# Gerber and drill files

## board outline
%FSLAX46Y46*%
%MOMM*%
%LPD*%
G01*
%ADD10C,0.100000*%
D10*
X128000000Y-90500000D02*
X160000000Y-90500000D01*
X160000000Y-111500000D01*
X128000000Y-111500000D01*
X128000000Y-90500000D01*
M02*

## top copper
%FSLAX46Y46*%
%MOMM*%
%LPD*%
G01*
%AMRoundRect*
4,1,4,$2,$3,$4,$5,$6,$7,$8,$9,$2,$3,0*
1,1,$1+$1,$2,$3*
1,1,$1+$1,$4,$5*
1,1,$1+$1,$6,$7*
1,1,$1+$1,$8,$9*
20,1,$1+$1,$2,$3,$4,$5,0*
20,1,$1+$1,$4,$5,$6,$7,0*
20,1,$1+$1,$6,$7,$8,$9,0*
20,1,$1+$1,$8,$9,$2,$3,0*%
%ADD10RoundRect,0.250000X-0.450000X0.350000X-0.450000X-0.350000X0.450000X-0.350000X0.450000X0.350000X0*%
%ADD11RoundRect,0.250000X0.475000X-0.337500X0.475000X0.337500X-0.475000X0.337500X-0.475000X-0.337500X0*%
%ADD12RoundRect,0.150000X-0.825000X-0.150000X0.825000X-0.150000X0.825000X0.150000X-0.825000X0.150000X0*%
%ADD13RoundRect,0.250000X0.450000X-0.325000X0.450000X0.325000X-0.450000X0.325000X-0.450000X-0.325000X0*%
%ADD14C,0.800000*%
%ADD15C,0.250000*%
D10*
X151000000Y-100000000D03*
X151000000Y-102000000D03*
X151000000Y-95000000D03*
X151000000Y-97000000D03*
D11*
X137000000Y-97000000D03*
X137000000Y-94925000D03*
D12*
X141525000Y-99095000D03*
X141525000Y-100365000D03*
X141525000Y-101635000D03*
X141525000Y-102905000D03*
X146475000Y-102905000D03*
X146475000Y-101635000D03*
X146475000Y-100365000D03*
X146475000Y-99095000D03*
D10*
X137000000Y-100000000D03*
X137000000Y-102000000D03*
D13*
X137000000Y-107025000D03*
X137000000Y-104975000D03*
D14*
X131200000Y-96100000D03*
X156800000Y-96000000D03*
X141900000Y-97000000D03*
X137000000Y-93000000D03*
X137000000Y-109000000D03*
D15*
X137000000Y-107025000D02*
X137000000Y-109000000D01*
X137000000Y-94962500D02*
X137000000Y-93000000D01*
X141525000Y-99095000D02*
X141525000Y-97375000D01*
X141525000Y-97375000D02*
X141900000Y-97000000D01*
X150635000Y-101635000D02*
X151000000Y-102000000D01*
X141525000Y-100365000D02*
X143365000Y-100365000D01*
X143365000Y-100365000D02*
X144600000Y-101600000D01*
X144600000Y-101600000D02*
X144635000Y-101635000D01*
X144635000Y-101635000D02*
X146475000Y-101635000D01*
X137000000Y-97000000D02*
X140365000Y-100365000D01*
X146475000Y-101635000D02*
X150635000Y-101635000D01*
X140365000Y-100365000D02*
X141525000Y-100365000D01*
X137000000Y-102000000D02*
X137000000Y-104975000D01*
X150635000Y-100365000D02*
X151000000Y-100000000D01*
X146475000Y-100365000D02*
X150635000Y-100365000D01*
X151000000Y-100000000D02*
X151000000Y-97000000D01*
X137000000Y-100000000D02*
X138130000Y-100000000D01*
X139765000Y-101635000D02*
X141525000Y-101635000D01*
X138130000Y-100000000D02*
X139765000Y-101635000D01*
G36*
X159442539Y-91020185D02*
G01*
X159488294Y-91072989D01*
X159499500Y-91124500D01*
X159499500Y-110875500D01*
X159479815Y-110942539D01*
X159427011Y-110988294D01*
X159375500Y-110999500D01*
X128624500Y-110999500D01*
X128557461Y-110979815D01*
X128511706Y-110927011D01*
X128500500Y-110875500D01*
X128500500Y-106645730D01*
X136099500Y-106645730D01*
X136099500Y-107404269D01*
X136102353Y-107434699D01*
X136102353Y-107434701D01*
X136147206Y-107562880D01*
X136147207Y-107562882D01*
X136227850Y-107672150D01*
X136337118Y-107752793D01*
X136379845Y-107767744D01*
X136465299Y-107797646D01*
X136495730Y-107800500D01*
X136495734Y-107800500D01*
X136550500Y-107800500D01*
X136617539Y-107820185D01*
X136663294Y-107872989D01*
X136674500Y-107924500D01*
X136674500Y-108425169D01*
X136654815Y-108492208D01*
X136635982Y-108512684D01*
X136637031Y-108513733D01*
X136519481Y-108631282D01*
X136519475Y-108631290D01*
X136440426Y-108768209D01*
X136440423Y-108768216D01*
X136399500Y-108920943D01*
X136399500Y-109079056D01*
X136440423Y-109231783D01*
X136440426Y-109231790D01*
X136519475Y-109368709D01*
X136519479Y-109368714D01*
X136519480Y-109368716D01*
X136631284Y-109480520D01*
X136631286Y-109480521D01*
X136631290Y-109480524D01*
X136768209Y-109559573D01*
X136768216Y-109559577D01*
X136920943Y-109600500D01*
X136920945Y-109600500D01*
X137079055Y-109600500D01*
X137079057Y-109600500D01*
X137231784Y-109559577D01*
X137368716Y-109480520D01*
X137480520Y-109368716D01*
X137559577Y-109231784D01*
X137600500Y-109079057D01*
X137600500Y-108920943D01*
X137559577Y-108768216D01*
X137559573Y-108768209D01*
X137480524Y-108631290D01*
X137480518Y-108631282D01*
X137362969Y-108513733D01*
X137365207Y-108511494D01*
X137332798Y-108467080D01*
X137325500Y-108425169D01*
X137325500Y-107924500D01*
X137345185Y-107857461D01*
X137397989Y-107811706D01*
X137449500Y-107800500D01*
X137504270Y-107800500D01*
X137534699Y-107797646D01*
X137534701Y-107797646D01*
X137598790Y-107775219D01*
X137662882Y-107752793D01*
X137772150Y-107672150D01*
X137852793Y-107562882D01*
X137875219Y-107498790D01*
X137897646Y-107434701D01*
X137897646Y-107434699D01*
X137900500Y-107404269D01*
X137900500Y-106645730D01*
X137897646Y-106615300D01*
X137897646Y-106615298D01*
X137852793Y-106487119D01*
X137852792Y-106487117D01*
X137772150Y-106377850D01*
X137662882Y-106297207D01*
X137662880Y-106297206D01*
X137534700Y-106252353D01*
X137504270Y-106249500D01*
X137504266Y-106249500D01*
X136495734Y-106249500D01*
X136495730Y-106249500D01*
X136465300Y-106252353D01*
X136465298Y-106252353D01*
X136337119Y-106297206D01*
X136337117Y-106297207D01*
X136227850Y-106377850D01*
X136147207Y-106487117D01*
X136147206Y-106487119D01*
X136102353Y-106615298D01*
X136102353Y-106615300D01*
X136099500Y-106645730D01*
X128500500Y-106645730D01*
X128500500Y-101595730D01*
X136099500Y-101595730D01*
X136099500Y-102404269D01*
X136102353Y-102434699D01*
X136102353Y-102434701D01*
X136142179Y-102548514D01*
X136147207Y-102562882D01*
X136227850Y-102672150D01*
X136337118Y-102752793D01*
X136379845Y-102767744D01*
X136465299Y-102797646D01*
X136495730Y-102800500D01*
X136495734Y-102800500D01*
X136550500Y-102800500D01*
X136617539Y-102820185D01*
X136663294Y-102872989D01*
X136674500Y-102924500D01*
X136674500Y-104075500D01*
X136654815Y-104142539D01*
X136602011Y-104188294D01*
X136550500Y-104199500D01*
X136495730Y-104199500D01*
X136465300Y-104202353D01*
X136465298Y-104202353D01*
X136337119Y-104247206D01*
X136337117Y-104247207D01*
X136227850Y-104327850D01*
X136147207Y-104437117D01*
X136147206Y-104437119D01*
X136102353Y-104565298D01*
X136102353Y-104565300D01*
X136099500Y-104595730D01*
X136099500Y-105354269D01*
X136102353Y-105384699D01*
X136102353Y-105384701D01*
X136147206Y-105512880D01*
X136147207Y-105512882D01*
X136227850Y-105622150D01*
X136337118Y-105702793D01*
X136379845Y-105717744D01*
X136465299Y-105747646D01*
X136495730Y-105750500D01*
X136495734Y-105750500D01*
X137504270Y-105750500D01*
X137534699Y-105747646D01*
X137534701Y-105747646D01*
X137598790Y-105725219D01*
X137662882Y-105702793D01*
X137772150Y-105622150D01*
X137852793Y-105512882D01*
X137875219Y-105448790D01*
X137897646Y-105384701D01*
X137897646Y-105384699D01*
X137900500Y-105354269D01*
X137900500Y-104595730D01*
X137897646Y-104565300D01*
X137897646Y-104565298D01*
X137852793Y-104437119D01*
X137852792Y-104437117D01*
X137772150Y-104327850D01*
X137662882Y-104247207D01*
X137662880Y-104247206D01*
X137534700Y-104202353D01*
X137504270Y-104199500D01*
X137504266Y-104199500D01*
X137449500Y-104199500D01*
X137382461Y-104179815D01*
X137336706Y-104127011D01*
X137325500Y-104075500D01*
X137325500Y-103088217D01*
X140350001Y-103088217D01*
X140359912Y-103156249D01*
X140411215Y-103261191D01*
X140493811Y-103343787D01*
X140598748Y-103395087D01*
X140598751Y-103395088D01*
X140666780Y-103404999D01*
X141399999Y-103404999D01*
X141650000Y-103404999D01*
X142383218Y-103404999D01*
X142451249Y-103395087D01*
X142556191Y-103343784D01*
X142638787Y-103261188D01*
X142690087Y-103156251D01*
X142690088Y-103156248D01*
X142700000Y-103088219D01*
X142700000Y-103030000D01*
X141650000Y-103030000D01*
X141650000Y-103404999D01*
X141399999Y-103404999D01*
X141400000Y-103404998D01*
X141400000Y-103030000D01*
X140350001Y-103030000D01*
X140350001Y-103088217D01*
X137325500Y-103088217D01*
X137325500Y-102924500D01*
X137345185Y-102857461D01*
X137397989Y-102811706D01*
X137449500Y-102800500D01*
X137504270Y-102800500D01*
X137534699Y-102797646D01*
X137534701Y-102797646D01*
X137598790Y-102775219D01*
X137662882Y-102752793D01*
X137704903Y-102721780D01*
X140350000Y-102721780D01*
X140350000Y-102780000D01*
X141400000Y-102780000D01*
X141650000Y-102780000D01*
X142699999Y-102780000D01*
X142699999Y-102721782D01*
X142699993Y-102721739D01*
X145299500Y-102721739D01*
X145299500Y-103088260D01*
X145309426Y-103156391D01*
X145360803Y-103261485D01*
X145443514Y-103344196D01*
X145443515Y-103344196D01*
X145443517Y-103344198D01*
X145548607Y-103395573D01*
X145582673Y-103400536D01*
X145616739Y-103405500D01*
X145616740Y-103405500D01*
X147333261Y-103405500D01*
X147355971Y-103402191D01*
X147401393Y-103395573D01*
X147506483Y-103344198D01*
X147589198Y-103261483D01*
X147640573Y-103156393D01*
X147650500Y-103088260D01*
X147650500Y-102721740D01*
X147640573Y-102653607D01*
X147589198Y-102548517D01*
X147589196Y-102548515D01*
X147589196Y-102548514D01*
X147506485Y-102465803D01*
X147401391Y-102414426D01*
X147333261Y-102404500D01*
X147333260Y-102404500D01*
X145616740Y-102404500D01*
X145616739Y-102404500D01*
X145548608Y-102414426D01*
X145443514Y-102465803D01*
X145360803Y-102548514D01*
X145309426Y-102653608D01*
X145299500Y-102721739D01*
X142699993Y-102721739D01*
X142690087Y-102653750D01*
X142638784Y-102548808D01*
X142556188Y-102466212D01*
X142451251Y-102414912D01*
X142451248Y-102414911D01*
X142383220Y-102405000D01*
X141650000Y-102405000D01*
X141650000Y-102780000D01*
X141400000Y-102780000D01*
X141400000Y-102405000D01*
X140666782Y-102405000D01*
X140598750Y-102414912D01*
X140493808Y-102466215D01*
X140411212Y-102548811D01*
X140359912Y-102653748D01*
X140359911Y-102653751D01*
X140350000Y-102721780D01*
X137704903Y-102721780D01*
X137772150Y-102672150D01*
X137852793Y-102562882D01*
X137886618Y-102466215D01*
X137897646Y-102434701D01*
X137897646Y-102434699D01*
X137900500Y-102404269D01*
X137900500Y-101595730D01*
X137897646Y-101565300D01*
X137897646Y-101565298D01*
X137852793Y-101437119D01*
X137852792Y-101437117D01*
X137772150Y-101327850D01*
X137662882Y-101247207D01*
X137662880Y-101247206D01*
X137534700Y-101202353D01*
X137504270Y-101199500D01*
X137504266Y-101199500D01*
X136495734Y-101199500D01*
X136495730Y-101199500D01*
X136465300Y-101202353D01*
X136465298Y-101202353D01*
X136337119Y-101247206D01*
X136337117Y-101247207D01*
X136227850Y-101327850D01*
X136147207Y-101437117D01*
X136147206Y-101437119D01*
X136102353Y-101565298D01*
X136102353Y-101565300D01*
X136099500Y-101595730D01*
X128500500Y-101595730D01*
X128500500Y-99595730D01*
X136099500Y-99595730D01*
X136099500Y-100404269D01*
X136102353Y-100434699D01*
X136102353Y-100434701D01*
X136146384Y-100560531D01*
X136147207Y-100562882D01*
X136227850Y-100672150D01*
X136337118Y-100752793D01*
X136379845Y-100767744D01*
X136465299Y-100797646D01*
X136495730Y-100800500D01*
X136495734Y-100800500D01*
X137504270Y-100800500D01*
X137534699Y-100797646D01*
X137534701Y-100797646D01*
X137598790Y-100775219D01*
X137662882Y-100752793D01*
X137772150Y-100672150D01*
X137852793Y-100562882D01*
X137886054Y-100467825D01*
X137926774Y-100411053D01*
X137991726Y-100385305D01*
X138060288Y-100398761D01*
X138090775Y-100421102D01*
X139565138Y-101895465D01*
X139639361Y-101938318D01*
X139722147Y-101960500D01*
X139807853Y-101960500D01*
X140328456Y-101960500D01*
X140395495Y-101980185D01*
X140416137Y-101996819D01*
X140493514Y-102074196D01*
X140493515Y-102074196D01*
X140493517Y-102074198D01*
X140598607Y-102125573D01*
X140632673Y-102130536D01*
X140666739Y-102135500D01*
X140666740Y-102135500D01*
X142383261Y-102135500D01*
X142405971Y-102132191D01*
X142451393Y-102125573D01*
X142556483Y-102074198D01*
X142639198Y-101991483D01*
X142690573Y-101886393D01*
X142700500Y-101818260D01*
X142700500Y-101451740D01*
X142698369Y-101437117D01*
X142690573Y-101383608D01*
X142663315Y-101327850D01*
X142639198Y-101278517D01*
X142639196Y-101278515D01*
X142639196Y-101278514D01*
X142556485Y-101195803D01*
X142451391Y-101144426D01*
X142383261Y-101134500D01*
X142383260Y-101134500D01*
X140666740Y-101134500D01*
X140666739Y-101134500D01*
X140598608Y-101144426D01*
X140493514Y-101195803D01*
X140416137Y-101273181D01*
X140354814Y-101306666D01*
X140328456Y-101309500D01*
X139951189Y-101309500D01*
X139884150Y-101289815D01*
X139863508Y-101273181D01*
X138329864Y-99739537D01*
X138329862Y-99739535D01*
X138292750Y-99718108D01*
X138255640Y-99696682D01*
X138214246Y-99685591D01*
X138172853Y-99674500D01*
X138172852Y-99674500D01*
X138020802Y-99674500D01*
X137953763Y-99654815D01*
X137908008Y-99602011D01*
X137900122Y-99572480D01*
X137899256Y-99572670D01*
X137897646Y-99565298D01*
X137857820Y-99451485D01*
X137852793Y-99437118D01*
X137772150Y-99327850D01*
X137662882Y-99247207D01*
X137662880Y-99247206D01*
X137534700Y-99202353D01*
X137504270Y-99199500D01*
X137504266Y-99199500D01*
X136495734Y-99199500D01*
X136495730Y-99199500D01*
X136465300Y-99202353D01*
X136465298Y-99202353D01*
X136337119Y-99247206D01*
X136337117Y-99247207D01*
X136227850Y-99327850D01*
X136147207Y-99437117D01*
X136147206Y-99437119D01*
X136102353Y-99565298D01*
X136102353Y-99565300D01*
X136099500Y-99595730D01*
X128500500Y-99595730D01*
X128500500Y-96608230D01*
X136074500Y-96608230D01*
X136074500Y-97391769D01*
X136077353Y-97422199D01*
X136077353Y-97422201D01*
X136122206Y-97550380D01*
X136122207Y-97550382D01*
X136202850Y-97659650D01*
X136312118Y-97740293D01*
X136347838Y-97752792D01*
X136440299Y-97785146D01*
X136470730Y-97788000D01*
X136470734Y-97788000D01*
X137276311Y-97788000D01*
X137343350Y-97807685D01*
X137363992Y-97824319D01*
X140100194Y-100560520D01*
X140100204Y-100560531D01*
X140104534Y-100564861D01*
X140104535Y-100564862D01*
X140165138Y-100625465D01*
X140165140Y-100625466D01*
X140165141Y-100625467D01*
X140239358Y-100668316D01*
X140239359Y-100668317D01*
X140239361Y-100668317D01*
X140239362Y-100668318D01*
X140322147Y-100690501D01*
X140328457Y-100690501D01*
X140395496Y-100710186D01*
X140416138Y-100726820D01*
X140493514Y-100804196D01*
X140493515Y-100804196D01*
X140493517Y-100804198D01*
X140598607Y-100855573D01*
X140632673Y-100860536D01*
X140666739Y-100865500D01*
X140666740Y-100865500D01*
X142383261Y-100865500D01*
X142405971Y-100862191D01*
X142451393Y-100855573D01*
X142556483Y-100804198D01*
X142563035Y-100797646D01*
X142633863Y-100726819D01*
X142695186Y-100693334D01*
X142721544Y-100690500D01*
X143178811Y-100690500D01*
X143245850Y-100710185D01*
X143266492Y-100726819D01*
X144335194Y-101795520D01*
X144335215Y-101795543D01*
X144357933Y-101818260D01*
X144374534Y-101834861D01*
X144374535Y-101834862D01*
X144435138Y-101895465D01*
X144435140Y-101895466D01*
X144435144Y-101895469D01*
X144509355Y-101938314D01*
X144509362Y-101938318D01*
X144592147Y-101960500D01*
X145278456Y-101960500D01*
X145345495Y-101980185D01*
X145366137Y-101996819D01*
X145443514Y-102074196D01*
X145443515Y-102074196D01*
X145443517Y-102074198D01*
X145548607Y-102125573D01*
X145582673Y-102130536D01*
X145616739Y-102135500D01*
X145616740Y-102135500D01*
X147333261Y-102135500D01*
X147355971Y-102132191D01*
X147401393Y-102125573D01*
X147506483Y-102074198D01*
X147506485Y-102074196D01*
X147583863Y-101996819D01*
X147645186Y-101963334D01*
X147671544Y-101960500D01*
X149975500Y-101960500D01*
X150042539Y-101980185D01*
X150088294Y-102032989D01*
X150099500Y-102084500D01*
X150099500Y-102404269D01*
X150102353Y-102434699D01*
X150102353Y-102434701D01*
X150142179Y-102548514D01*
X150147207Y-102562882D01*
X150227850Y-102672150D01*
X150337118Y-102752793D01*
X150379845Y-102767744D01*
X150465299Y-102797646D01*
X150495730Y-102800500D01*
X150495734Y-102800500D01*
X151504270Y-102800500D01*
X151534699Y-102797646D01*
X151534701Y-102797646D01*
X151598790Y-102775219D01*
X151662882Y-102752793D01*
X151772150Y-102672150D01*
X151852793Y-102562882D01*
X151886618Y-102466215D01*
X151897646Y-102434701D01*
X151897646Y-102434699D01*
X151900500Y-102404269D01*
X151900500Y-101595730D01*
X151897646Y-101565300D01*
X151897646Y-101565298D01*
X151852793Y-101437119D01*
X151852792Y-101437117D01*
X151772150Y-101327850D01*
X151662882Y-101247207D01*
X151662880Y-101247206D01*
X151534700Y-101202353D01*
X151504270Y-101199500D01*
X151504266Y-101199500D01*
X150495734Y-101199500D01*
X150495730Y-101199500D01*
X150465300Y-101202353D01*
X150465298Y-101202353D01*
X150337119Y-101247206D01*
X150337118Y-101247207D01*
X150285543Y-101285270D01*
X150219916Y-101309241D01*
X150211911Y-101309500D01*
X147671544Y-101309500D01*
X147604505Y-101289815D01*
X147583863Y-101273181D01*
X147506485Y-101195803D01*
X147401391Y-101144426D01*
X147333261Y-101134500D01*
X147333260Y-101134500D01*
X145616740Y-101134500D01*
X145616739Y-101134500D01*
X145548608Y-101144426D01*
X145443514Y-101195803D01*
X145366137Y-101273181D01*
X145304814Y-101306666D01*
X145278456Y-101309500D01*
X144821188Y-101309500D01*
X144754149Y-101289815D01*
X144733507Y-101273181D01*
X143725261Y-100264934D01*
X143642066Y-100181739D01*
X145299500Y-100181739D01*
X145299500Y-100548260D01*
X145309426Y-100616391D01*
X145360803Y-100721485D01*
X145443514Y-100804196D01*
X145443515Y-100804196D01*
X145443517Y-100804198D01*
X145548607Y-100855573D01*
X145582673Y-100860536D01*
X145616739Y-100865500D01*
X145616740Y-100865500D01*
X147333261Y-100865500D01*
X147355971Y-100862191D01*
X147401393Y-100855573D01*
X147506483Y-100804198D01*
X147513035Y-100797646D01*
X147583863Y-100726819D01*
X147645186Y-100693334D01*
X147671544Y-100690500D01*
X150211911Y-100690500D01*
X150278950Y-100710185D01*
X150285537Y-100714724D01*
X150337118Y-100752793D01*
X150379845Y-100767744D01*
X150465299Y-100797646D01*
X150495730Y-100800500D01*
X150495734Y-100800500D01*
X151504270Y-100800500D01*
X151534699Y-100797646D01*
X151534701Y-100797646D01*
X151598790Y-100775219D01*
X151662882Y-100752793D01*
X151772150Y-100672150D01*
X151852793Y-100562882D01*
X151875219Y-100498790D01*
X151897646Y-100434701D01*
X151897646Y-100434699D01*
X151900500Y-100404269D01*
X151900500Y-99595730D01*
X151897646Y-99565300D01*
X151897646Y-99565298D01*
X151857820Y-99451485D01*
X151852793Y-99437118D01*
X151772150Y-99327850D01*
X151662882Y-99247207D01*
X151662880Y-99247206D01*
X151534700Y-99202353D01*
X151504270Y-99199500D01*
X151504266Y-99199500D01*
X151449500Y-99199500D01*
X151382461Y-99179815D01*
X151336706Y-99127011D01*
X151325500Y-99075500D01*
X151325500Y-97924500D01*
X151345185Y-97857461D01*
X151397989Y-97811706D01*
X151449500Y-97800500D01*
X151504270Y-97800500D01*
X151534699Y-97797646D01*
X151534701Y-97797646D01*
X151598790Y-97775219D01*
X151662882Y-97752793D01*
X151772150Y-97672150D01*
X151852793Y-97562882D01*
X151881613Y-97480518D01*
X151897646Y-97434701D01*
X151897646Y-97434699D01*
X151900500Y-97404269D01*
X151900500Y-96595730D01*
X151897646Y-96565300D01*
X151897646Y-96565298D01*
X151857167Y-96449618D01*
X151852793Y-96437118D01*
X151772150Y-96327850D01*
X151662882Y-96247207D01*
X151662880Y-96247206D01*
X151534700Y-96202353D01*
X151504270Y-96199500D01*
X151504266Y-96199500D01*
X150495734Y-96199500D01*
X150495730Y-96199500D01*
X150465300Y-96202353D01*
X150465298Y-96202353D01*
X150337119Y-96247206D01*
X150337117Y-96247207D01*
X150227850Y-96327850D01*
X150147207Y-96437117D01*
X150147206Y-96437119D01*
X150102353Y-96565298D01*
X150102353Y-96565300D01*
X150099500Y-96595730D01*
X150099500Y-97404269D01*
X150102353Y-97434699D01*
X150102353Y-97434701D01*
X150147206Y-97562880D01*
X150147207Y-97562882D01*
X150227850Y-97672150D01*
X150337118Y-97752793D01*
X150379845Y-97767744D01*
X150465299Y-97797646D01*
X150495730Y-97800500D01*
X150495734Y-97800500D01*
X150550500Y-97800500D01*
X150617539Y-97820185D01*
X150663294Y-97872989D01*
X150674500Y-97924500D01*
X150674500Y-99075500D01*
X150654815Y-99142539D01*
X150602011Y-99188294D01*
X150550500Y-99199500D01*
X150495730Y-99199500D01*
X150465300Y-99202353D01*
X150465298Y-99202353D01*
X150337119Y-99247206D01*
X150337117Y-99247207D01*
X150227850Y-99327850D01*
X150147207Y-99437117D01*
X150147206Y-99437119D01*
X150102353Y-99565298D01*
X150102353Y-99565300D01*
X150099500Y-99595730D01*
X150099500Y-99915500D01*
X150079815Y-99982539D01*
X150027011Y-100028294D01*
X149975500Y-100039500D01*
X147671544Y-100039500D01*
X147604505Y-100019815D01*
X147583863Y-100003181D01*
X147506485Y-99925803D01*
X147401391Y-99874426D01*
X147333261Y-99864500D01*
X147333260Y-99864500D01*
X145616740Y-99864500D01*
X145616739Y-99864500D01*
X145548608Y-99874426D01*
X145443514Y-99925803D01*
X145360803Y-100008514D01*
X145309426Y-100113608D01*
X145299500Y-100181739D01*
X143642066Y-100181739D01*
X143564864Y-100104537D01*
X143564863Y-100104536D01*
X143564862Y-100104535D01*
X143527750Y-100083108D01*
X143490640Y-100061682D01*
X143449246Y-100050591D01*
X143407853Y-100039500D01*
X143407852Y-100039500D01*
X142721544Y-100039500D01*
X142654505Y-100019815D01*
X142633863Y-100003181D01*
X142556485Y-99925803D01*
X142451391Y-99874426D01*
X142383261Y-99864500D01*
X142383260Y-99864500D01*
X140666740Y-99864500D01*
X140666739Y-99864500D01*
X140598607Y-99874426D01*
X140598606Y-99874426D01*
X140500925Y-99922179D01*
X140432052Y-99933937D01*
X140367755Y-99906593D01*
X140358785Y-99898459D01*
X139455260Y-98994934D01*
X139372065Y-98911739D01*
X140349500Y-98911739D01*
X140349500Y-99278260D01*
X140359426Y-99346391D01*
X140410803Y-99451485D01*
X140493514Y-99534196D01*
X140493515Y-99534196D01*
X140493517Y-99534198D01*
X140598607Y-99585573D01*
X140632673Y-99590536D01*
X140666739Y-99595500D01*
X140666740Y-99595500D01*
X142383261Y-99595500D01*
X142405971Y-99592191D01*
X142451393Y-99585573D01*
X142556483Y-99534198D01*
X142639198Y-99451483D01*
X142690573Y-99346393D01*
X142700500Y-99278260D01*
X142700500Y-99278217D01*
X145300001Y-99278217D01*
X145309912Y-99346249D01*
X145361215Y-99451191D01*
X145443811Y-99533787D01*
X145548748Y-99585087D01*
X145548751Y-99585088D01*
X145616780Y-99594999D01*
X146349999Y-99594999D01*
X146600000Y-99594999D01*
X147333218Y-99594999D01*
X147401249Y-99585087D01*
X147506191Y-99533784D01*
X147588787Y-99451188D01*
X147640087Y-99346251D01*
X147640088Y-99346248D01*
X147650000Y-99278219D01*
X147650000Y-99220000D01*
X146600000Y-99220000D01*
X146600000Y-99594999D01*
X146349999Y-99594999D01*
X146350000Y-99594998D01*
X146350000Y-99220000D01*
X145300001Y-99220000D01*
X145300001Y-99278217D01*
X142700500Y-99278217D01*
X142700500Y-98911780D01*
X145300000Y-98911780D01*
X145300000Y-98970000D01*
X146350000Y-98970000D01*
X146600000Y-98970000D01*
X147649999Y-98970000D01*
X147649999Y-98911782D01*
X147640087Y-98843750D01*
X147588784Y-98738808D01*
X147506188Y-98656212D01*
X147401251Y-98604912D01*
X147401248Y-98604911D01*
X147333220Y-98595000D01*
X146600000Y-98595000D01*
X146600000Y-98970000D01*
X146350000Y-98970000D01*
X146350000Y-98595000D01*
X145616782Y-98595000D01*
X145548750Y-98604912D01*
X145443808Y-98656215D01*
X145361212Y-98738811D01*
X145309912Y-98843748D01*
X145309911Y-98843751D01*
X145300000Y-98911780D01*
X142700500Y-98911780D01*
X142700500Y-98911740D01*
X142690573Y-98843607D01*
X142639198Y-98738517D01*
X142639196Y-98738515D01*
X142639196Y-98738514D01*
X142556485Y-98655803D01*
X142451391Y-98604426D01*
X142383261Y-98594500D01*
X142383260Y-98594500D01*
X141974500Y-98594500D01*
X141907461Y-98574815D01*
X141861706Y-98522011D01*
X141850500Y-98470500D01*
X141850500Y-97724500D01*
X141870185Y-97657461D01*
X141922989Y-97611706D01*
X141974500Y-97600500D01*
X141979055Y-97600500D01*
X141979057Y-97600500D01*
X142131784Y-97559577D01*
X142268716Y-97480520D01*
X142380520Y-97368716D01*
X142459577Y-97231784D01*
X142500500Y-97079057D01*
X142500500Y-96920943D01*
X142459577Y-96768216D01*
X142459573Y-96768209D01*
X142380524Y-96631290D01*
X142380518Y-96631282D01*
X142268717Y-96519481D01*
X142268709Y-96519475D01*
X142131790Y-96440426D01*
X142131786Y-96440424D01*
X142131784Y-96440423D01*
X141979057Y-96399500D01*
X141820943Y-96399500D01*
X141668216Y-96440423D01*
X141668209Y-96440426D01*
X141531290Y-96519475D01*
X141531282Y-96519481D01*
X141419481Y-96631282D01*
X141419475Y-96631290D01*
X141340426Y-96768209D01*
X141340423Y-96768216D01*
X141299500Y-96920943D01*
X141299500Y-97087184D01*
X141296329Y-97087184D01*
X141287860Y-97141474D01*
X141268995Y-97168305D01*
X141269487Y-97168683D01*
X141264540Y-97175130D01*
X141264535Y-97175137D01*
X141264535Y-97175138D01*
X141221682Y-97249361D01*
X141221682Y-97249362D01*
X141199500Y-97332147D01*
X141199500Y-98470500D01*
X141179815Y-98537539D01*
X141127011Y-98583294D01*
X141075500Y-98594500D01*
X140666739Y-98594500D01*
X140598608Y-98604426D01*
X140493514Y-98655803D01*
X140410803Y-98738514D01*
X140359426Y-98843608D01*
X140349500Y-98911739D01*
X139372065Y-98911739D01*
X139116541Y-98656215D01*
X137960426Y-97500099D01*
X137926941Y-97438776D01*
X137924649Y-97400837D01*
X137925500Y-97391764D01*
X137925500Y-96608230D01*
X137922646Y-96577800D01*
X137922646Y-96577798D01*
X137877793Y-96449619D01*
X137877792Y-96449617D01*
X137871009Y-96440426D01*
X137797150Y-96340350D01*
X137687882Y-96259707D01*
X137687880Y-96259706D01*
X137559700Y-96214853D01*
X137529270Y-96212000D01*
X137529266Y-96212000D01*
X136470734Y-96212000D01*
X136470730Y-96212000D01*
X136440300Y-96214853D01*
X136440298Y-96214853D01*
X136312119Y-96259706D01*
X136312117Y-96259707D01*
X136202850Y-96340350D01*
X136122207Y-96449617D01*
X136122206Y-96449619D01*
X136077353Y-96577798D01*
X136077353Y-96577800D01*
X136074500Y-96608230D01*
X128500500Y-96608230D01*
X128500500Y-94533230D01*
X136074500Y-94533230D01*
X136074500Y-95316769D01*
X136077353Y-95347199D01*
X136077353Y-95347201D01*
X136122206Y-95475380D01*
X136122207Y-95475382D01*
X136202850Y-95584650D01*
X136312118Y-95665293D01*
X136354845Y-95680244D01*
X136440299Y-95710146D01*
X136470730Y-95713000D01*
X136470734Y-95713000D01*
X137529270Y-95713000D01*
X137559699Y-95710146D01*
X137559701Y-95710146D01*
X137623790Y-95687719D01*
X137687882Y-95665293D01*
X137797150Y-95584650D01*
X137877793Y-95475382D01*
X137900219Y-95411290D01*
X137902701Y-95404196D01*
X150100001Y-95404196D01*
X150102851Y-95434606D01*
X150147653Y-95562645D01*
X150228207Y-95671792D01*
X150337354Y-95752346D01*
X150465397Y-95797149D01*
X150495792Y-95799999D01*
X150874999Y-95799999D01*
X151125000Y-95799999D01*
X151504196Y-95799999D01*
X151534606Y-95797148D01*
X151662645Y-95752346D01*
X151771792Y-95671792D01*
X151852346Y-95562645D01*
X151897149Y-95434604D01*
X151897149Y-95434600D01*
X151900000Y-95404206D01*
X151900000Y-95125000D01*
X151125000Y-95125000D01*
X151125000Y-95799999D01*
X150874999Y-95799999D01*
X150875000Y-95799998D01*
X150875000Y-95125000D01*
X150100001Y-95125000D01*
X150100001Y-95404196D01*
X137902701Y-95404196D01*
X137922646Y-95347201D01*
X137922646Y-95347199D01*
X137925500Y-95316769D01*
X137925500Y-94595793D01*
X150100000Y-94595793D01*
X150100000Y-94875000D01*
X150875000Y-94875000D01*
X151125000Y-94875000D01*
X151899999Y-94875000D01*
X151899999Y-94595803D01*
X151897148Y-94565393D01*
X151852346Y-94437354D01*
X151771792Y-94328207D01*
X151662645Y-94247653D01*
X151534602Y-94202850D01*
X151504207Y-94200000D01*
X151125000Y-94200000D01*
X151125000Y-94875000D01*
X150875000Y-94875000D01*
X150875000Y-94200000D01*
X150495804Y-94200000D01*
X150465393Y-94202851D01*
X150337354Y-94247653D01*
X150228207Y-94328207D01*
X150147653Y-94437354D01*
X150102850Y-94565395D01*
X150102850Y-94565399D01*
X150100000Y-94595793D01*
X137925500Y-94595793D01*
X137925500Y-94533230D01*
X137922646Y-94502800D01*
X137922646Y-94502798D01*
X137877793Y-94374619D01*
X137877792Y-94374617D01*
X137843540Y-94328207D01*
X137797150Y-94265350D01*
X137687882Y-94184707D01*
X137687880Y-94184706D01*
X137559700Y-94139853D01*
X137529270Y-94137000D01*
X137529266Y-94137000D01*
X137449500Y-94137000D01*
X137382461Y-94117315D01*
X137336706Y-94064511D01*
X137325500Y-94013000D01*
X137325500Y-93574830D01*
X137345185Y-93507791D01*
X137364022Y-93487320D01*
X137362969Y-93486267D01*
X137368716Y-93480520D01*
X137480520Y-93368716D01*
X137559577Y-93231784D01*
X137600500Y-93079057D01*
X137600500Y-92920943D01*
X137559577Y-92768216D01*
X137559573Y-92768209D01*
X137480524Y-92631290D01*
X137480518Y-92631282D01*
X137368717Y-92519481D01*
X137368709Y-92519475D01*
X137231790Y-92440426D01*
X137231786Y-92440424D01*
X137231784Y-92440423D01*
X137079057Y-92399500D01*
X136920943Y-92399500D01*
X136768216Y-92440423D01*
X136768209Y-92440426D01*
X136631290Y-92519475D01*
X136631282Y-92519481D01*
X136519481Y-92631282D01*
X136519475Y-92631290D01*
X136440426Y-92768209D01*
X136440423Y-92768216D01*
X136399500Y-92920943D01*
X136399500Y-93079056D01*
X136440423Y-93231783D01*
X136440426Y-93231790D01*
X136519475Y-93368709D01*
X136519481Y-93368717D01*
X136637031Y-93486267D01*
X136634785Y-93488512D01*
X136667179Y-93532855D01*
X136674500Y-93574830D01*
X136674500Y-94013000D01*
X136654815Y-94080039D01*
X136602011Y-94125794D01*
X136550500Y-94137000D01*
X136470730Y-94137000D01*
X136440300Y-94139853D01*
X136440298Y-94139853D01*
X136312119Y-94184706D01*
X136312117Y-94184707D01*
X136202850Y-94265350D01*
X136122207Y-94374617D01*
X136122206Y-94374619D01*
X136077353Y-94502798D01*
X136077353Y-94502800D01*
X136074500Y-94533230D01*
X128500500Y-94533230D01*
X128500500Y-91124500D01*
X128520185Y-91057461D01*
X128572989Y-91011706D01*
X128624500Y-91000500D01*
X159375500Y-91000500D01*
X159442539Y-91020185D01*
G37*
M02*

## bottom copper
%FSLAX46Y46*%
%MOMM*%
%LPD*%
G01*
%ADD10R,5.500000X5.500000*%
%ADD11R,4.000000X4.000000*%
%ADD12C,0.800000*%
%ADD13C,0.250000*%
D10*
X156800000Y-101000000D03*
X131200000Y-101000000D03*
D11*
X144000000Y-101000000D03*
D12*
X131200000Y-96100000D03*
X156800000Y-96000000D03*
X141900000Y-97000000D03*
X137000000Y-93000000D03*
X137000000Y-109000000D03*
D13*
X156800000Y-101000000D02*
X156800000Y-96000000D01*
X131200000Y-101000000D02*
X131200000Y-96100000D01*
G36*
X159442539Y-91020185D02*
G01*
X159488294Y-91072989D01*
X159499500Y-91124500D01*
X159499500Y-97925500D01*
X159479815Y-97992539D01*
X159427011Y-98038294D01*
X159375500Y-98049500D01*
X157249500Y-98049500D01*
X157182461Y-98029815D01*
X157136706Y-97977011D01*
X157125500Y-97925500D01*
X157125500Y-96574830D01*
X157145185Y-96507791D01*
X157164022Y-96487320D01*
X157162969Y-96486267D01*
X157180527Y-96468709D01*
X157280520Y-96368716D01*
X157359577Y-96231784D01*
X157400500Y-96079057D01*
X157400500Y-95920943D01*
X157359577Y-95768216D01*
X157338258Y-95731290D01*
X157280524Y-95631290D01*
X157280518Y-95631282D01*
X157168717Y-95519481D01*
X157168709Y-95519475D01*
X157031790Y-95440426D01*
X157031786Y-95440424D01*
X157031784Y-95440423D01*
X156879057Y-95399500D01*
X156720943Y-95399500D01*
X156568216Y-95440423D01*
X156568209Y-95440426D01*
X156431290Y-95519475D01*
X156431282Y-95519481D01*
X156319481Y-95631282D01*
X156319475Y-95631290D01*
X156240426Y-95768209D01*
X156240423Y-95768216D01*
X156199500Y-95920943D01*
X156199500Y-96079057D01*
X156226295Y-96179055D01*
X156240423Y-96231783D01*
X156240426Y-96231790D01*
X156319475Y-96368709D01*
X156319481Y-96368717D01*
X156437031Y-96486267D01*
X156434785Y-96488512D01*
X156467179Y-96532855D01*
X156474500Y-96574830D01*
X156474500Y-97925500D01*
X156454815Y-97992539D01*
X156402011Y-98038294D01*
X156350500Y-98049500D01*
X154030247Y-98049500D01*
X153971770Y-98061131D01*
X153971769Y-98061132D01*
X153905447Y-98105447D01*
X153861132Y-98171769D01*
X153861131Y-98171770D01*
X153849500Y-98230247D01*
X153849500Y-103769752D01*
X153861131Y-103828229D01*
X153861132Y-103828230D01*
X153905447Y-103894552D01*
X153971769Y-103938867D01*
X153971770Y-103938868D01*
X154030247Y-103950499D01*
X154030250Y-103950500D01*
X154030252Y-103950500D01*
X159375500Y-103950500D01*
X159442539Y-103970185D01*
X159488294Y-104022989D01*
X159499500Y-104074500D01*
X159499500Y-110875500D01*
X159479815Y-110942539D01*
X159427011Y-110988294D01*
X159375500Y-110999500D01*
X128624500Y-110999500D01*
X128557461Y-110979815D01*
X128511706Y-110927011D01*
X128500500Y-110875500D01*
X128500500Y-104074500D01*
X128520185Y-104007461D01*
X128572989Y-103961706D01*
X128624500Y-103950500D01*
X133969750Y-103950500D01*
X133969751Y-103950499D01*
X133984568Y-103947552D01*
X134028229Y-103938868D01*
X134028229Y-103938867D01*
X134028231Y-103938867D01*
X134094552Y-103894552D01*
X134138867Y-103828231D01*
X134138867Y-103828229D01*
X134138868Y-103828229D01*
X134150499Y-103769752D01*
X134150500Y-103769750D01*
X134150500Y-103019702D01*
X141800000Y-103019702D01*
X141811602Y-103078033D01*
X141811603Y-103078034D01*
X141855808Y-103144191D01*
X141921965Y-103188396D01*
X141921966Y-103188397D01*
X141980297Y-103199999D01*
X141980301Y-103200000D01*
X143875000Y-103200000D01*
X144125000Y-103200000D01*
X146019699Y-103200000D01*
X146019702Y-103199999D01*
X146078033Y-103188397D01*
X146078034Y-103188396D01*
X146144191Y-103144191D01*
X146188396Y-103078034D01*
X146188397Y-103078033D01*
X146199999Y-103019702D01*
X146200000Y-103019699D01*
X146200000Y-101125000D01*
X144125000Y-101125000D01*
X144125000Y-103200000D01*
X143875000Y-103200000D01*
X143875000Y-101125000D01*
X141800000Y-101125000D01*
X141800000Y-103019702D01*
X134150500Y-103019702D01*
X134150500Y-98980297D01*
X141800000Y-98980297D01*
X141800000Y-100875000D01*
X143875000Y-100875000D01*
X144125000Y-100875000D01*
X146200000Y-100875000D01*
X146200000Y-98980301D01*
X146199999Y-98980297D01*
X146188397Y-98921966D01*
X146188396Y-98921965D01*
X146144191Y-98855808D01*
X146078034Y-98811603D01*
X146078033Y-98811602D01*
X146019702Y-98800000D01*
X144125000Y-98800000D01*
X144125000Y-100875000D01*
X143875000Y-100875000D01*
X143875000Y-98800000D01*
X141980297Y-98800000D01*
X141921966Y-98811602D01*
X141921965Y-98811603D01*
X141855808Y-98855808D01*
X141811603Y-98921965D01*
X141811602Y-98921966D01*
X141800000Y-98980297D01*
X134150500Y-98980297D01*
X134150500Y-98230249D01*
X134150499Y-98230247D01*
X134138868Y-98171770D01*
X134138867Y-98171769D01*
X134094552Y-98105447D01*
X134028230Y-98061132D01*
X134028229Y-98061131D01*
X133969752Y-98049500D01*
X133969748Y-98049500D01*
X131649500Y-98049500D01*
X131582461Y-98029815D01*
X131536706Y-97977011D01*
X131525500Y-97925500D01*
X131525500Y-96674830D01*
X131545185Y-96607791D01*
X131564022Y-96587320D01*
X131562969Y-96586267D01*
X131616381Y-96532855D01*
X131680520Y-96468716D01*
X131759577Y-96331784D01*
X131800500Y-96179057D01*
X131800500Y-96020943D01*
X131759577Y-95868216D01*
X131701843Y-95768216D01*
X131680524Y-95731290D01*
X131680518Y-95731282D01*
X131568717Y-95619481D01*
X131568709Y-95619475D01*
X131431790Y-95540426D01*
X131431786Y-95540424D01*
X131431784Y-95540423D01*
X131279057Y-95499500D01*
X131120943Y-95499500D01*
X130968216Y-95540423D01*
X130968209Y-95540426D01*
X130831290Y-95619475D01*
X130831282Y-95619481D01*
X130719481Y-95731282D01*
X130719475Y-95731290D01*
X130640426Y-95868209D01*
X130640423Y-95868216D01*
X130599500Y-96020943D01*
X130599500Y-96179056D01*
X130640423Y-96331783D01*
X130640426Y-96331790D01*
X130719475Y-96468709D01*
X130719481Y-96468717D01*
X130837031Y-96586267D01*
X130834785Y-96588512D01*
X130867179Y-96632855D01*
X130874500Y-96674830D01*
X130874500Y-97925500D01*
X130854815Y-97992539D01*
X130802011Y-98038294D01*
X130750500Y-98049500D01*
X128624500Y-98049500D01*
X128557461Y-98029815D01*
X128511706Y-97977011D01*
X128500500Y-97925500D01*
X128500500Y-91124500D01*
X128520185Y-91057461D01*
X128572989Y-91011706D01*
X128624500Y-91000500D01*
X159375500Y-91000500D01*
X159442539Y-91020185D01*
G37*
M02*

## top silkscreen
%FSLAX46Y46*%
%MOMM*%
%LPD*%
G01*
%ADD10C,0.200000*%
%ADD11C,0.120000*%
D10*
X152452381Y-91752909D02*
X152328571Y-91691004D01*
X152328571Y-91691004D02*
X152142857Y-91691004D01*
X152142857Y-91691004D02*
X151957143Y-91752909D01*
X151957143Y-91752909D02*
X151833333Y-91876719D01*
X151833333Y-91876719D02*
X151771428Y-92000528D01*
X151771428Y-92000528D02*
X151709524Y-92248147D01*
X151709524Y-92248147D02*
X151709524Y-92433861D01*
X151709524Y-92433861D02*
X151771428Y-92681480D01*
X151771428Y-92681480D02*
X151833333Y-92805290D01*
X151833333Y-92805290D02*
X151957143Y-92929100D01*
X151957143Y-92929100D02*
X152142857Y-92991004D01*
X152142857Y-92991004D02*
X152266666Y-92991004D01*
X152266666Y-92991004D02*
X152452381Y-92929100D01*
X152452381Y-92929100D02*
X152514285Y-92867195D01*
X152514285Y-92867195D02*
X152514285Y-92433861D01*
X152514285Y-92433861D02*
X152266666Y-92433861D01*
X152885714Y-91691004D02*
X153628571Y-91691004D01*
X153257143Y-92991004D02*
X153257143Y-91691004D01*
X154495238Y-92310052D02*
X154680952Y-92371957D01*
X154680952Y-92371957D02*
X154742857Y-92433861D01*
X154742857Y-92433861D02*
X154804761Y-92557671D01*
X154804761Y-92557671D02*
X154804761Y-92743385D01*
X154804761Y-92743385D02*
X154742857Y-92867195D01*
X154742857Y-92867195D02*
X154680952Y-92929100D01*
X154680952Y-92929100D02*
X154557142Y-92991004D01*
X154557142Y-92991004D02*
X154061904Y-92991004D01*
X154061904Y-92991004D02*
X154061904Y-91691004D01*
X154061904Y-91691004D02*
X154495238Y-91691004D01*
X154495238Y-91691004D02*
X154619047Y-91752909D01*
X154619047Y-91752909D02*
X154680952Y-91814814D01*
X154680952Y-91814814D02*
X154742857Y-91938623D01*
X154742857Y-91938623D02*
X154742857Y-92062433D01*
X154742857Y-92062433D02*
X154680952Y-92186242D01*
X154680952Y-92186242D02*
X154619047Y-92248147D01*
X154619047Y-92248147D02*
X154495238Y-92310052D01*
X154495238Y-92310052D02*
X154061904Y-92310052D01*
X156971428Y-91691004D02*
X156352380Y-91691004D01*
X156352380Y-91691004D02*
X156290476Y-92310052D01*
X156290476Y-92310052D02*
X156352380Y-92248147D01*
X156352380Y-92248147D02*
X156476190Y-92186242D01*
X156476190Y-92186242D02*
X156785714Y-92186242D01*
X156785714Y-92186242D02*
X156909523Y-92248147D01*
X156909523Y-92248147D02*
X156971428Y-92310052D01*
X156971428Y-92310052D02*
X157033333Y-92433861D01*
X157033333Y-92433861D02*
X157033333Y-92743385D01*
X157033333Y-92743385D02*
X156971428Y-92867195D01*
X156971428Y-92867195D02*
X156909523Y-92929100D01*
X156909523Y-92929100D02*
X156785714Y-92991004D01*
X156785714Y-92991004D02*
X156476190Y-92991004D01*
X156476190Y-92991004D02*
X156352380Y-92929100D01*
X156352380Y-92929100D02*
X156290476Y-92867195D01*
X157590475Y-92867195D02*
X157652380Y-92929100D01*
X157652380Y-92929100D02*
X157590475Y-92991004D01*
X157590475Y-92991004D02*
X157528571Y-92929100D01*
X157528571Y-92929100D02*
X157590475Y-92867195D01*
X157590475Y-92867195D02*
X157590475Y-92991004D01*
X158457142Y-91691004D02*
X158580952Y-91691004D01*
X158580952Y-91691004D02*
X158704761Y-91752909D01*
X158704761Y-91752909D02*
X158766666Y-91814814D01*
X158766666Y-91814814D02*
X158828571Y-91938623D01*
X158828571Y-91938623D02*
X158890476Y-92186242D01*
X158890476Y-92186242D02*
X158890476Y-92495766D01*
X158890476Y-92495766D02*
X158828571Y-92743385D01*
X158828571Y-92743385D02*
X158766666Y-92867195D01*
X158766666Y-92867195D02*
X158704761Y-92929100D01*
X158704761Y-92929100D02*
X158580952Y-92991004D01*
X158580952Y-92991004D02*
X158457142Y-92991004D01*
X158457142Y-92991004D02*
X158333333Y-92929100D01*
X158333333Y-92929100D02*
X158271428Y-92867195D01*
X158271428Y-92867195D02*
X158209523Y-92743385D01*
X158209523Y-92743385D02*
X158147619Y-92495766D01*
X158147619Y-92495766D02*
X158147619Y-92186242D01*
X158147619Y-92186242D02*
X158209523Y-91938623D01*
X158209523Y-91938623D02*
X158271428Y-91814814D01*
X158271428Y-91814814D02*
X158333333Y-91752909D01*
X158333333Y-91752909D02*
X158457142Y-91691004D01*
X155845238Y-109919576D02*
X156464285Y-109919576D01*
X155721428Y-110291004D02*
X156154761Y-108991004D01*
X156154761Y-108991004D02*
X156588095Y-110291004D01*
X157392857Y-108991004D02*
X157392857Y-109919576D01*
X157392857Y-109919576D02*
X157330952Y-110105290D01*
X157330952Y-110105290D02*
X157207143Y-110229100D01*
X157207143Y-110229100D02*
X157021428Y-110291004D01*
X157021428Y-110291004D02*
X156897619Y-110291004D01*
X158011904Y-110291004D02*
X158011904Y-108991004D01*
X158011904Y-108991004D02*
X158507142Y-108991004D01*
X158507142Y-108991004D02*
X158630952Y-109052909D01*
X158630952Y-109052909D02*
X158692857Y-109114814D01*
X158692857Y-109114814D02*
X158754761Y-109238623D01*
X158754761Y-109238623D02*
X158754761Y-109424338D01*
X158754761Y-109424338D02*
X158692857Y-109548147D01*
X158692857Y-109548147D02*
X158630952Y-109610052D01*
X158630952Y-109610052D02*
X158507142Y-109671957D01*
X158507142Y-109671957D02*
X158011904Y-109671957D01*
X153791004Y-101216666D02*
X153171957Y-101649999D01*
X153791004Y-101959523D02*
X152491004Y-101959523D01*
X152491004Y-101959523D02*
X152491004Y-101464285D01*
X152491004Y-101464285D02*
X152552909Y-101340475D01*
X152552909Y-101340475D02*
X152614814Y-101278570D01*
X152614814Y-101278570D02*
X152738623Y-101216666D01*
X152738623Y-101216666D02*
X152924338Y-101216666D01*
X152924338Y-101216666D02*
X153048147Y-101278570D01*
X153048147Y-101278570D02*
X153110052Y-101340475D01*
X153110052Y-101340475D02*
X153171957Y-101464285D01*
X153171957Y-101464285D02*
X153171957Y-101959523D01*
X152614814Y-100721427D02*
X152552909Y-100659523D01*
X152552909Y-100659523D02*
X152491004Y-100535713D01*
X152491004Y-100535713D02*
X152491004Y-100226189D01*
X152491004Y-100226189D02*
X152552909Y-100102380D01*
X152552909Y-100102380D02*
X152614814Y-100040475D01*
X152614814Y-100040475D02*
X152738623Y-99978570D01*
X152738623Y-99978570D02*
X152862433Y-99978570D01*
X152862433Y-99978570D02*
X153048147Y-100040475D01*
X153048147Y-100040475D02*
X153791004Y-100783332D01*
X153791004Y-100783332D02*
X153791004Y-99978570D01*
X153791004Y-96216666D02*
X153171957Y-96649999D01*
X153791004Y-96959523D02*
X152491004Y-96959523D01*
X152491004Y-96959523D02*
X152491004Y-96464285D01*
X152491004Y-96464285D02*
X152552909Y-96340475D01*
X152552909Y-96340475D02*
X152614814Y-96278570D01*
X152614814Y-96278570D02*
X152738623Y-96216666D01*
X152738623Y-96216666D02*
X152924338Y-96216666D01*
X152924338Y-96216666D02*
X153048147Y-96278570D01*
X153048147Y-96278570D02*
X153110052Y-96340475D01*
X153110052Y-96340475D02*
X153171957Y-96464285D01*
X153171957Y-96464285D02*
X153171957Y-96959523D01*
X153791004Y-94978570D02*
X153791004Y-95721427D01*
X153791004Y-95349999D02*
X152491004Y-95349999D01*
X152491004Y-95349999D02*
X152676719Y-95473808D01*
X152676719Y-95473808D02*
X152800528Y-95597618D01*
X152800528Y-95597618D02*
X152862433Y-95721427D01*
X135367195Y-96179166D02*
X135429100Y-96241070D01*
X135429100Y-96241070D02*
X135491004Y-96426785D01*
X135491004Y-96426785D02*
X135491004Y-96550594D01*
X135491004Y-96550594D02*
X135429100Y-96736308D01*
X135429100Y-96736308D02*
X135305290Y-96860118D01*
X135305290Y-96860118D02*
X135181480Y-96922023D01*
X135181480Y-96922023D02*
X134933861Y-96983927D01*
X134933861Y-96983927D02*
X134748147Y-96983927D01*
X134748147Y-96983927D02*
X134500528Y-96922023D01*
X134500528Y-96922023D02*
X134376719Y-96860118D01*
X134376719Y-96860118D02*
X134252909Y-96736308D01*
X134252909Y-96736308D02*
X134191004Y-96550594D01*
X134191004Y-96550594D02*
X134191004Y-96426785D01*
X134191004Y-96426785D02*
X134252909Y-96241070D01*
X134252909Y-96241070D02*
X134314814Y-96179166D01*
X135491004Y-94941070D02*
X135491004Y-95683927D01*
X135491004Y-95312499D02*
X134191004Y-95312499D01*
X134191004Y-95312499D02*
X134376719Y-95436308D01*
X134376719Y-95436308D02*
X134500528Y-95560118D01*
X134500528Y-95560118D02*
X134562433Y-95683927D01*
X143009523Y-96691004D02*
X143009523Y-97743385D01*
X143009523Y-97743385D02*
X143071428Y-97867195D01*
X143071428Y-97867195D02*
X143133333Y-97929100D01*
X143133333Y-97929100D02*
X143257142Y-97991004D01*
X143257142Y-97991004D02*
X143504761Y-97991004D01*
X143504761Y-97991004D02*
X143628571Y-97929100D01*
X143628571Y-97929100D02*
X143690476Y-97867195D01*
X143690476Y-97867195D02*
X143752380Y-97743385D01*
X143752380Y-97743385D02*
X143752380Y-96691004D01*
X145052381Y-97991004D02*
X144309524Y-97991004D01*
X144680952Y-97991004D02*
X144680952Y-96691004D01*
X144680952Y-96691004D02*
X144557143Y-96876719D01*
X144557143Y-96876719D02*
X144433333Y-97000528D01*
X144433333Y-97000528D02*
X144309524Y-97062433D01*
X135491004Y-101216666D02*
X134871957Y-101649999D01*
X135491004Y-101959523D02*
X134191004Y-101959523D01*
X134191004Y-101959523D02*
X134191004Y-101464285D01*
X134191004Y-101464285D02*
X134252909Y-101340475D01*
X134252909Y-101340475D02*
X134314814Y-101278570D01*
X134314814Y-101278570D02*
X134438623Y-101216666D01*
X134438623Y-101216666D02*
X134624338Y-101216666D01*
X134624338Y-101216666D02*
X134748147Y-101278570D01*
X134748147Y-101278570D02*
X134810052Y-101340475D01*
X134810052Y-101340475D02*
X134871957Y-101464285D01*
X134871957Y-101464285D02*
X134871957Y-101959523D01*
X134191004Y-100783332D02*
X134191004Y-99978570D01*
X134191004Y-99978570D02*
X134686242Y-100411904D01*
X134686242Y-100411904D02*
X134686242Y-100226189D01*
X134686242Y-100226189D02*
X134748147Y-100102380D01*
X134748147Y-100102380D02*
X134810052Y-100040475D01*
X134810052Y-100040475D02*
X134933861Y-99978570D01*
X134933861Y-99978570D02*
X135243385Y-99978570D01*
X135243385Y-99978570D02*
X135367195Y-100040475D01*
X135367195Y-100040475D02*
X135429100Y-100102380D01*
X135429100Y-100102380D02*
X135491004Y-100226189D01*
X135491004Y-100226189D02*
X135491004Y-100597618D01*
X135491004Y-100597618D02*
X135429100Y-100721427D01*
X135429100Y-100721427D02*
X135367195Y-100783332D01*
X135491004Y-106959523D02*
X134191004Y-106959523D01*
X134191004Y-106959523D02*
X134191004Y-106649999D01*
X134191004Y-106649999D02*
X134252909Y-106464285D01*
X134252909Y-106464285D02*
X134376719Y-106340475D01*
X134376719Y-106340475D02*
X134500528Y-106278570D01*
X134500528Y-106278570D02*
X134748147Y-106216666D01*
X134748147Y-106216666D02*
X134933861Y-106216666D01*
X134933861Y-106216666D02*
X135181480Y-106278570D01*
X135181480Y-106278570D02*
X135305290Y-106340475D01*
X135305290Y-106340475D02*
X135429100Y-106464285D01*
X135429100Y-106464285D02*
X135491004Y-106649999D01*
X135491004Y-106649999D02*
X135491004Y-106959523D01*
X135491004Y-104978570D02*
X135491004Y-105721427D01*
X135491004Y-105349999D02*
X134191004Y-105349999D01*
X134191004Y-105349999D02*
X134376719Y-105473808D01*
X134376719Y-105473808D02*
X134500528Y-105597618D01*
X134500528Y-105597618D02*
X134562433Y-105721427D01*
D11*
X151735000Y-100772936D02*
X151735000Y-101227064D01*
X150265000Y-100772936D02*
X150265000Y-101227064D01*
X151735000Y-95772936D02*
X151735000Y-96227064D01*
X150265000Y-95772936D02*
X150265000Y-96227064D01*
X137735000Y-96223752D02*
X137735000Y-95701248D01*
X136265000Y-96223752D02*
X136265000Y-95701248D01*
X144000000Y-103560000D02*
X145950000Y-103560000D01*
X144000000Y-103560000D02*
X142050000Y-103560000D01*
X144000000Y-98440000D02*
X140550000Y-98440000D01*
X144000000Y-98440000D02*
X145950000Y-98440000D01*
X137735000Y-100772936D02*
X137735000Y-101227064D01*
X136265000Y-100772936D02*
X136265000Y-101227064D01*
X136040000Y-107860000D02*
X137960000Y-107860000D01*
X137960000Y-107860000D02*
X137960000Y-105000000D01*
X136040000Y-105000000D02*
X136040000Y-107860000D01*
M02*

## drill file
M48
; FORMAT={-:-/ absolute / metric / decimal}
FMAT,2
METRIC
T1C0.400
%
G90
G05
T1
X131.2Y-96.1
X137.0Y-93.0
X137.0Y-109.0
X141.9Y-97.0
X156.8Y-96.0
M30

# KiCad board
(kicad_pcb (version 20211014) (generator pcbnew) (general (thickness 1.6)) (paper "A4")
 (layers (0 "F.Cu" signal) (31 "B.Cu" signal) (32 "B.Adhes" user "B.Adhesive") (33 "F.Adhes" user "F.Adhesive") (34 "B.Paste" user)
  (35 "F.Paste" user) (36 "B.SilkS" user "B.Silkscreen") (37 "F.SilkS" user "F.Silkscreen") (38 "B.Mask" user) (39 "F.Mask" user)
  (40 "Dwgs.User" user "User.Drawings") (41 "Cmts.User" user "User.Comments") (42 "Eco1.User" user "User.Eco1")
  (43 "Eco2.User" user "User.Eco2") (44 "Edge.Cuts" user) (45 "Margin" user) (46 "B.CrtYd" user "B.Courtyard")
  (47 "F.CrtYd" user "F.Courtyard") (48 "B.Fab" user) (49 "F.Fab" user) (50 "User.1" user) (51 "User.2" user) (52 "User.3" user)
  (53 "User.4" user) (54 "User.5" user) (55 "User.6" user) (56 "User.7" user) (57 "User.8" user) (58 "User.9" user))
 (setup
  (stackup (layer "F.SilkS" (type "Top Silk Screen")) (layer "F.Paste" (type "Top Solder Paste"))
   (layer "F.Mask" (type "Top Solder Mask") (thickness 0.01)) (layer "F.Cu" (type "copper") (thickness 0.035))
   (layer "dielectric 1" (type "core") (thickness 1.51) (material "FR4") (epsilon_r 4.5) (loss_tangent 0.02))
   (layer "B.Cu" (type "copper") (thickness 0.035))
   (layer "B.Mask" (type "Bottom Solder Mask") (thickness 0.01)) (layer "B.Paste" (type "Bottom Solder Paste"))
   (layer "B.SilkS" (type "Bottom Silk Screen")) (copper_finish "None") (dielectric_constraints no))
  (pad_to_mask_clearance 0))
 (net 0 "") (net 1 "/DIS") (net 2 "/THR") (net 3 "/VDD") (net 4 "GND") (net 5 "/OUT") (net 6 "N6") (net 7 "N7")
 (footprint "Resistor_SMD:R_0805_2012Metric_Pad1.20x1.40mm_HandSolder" (layer "F.Cu") (at 151 101 -90)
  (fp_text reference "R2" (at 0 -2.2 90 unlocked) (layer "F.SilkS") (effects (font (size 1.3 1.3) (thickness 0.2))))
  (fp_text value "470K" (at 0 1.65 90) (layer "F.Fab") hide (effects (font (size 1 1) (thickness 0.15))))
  (fp_line (start -0.227064 -0.735) (end 0.227064 -0.735) (layer "F.SilkS") (width 0.12))
  (fp_line (start -0.227064 0.735) (end 0.227064 0.735) (layer "F.SilkS") (width 0.12))
  (pad "1" smd roundrect (at -1 0 270) (size 1.2 1.4) (layers "F.Cu" "F.Paste" "F.Mask") (roundrect_rratio 0.2083333333) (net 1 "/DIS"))
  (pad "2" smd roundrect (at 1 0 270) (size 1.2 1.4) (layers "F.Cu" "F.Paste" "F.Mask") (roundrect_rratio 0.2083333333) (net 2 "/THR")))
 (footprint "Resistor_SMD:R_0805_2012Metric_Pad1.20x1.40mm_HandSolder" (layer "F.Cu") (at 151 96 -90)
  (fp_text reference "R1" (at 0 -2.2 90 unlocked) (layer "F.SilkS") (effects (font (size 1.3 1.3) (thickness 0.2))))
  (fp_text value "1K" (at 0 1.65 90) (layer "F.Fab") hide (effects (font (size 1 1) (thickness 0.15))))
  (fp_line (start -0.227064 -0.735) (end 0.227064 -0.735) (layer "F.SilkS") (width 0.12))
  (fp_line (start -0.227064 0.735) (end 0.227064 0.735) (layer "F.SilkS") (width 0.12))
  (pad "1" smd roundrect (at -1 0 270) (size 1.2 1.4) (layers "F.Cu" "F.Paste" "F.Mask") (roundrect_rratio 0.2083333333) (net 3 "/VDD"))
  (pad "2" smd roundrect (at 1 0 270) (size 1.2 1.4) (layers "F.Cu" "F.Paste" "F.Mask") (roundrect_rratio 0.2083333333) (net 1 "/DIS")))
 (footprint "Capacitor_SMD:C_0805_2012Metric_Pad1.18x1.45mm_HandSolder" (layer "F.Cu") (at 137 95.9625 90)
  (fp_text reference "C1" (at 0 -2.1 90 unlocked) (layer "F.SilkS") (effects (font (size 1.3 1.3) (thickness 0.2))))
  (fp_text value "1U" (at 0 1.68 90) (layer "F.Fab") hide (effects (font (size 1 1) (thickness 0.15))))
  (fp_line (start -0.261252 0.735) (end 0.261252 0.735) (layer "F.SilkS") (width 0.12))
  (fp_line (start -0.261252 -0.735) (end 0.261252 -0.735) (layer "F.SilkS") (width 0.12))
  (pad "1" smd roundrect (at -1.0375 0 90) (size 1.175 1.45) (layers "F.Cu" "F.Paste" "F.Mask") (roundrect_rratio 0.2127659574)
   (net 2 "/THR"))
  (pad "2" smd roundrect (at 1.0375 0 90) (size 1.175 1.45) (layers "F.Cu" "F.Paste" "F.Mask") (roundrect_rratio 0.2127659574) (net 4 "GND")))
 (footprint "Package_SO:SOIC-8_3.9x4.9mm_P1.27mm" (layer "F.Cu") (at 144 101)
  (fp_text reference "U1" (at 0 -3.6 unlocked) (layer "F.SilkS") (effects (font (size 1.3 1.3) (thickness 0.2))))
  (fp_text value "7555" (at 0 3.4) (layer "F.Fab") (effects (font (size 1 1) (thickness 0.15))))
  (fp_line (start 0 2.56) (end 1.95 2.56) (layer "F.SilkS") (width 0.12))
  (fp_line (start 0 2.56) (end -1.95 2.56) (layer "F.SilkS") (width 0.12))
  (fp_line (start 0 -2.56) (end -3.45 -2.56) (layer "F.SilkS") (width 0.12))
  (fp_line (start 0 -2.56) (end 1.95 -2.56) (layer "F.SilkS") (width 0.12))
  (pad "1" smd roundrect (at -2.475 -1.905) (size 1.95 0.6) (layers "F.Cu" "F.Paste" "F.Mask") (roundrect_rratio 0.25) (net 4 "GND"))
  (pad "2" smd roundrect (at -2.475 -0.635) (size 1.95 0.6) (layers "F.Cu" "F.Paste" "F.Mask") (roundrect_rratio 0.25) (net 2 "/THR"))
  (pad "3" smd roundrect (at -2.475 0.635) (size 1.95 0.6) (layers "F.Cu" "F.Paste" "F.Mask") (roundrect_rratio 0.25) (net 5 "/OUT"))
  (pad "4" smd roundrect (at -2.475 1.905) (size 1.95 0.6) (layers "F.Cu" "F.Paste" "F.Mask") (roundrect_rratio 0.25) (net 3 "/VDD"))
  (pad "5" smd roundrect (at 2.475 1.905) (size 1.95 0.6) (layers "F.Cu" "F.Paste" "F.Mask") (roundrect_rratio 0.25) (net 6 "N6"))
  (pad "6" smd roundrect (at 2.475 0.635) (size 1.95 0.6) (layers "F.Cu" "F.Paste" "F.Mask") (roundrect_rratio 0.25) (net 2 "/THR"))
  (pad "7" smd roundrect (at 2.475 -0.635) (size 1.95 0.6) (layers "F.Cu" "F.Paste" "F.Mask") (roundrect_rratio 0.25) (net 1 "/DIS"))
  (pad "8" smd roundrect (at 2.475 -1.905) (size 1.95 0.6) (layers "F.Cu" "F.Paste" "F.Mask") (roundrect_rratio 0.25) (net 3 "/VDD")))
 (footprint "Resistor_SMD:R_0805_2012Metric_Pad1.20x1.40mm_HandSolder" (layer "F.Cu") (at 137 101 -90)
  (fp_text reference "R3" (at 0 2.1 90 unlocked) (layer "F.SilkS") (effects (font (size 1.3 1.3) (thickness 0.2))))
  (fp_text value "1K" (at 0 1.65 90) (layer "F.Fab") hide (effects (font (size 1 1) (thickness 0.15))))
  (fp_line (start -0.227064 -0.735) (end 0.227064 -0.735) (layer "F.SilkS") (width 0.12))
  (fp_line (start -0.227064 0.735) (end 0.227064 0.735) (layer "F.SilkS") (width 0.12))
  (pad "1" smd roundrect (at -1 0 270) (size 1.2 1.4) (layers "F.Cu" "F.Paste" "F.Mask") (roundrect_rratio 0.2083333333) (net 5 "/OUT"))
  (pad "2" smd roundrect (at 1 0 270) (size 1.2 1.4) (layers "F.Cu" "F.Paste" "F.Mask") (roundrect_rratio 0.2083333333) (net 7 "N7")))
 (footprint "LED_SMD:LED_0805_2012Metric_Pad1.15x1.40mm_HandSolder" (layer "F.Cu") (at 137 106 90)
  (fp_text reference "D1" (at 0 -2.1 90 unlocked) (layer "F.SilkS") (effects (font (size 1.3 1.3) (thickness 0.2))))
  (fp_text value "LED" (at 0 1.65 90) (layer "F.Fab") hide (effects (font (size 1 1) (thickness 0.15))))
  (fp_line (start -1.86 -0.96) (end -1.86 0.96) (layer "F.SilkS") (width 0.12))
  (fp_line (start -1.86 0.96) (end 1 0.96) (layer "F.SilkS") (width 0.12))
  (fp_line (start 1 -0.96) (end -1.86 -0.96) (layer "F.SilkS") (width 0.12))
  (pad "1" smd roundrect (at -1.025 0 90) (size 1.15 1.4) (layers "F.Cu" "F.Paste" "F.Mask") (roundrect_rratio 0.2173913043) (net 4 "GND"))
  (pad "2" smd roundrect (at 1.025 0 90) (size 1.15 1.4) (layers "F.Cu" "F.Paste" "F.Mask") (roundrect_rratio 0.2173913043) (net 7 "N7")))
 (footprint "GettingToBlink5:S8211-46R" (layer "B.Cu") (at 144 101 180)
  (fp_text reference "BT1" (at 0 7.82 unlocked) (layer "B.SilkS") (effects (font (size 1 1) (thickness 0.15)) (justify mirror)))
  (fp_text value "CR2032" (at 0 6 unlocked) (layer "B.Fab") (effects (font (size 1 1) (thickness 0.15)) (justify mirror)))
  (pad "1" smd rect (at -12.8 0 180) (size 5.5 5.5) (layers "B.Cu" "B.Paste" "B.Mask") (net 3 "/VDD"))
  (pad "1" smd rect (at 12.8 0 180) (size 5.5 5.5) (layers "B.Cu" "B.Paste" "B.Mask") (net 3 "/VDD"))
  (pad "2" smd rect (at 0 0 180) (size 4 4) (layers "B.Cu" "B.Paste" "B.Mask") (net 4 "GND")))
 (gr_rect (start 160 111.5) (end 128 90.5) (layer "Edge.Cuts") (width 0.1) (fill none))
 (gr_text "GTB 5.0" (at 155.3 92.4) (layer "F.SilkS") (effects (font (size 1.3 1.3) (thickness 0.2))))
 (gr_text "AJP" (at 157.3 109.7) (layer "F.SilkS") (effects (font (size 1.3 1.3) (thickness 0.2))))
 (via (at 131.2 96.1) (size 0.8) (drill 0.4) (layers "F.Cu" "B.Cu") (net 3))
 (via (at 156.8 96) (size 0.8) (drill 0.4) (layers "F.Cu" "B.Cu") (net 3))
 (segment (start 156.8 101) (end 156.8 96) (width 0.25) (layer "B.Cu") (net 3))
 (segment (start 131.2 101) (end 131.2 96.1) (width 0.25) (layer "B.Cu") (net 3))
 (segment (start 137 107.025) (end 137 109) (width 0.25) (layer "F.Cu") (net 4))
 (segment (start 137 94.9625) (end 137 93) (width 0.25) (layer "F.Cu") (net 4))
 (segment (start 141.525 99.095) (end 141.525 97.375) (width 0.25) (layer "F.Cu") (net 4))
 (segment (start 141.525 97.375) (end 141.9 97) (width 0.25) (layer "F.Cu") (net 4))
 (via (at 141.9 97) (size 0.8) (drill 0.4) (layers "F.Cu" "B.Cu") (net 4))
 (via (at 137 93) (size 0.8) (drill 0.4) (layers "F.Cu" "B.Cu") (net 4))
 (via (at 137 109) (size 0.8) (drill 0.4) (layers "F.Cu" "B.Cu") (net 4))
 (segment (start 150.635 101.635) (end 151 102) (width 0.25) (layer "F.Cu") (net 2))
 (segment (start 141.525 100.365) (end 143.365 100.365) (width 0.25) (layer "F.Cu") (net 2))
 (segment (start 143.365 100.365) (end 144.6 101.6) (width 0.25) (layer "F.Cu") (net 2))
 (segment (start 144.6 101.6) (end 144.635 101.635) (width 0.25) (layer "F.Cu") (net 2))
 (segment (start 144.635 101.635) (end 146.475 101.635) (width 0.25) (layer "F.Cu") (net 2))
 (segment (start 137 97) (end 140.365 100.365) (width 0.25) (layer "F.Cu") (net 2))
 (segment (start 146.475 101.635) (end 150.635 101.635) (width 0.25) (layer "F.Cu") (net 2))
 (segment (start 140.365 100.365) (end 141.525 100.365) (width 0.25) (layer "F.Cu") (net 2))
 (segment (start 137 102) (end 137 104.975) (width 0.25) (layer "F.Cu") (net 7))
 (segment (start 150.635 100.365) (end 151 100) (width 0.25) (layer "F.Cu") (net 1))
 (segment (start 146.475 100.365) (end 150.635 100.365) (width 0.25) (layer "F.Cu") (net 1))
 (segment (start 151 100) (end 151 97) (width 0.25) (layer "F.Cu") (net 1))
 (segment (start 137 100) (end 138.13 100) (width 0.25) (layer "F.Cu") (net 5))
 (segment (start 139.765 101.635) (end 141.525 101.635) (width 0.25) (layer "F.Cu") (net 5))
 (segment (start 138.13 100) (end 139.765 101.635) (width 0.25) (layer "F.Cu") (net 5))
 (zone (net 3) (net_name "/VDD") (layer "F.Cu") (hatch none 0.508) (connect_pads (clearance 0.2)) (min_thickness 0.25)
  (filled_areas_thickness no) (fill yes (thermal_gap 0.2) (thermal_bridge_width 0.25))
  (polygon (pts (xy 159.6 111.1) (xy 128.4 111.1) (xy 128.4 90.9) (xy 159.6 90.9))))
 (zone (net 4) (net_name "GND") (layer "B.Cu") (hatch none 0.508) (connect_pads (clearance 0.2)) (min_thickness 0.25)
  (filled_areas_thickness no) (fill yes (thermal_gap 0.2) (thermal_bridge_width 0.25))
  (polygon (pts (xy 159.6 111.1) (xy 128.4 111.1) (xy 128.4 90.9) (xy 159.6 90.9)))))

